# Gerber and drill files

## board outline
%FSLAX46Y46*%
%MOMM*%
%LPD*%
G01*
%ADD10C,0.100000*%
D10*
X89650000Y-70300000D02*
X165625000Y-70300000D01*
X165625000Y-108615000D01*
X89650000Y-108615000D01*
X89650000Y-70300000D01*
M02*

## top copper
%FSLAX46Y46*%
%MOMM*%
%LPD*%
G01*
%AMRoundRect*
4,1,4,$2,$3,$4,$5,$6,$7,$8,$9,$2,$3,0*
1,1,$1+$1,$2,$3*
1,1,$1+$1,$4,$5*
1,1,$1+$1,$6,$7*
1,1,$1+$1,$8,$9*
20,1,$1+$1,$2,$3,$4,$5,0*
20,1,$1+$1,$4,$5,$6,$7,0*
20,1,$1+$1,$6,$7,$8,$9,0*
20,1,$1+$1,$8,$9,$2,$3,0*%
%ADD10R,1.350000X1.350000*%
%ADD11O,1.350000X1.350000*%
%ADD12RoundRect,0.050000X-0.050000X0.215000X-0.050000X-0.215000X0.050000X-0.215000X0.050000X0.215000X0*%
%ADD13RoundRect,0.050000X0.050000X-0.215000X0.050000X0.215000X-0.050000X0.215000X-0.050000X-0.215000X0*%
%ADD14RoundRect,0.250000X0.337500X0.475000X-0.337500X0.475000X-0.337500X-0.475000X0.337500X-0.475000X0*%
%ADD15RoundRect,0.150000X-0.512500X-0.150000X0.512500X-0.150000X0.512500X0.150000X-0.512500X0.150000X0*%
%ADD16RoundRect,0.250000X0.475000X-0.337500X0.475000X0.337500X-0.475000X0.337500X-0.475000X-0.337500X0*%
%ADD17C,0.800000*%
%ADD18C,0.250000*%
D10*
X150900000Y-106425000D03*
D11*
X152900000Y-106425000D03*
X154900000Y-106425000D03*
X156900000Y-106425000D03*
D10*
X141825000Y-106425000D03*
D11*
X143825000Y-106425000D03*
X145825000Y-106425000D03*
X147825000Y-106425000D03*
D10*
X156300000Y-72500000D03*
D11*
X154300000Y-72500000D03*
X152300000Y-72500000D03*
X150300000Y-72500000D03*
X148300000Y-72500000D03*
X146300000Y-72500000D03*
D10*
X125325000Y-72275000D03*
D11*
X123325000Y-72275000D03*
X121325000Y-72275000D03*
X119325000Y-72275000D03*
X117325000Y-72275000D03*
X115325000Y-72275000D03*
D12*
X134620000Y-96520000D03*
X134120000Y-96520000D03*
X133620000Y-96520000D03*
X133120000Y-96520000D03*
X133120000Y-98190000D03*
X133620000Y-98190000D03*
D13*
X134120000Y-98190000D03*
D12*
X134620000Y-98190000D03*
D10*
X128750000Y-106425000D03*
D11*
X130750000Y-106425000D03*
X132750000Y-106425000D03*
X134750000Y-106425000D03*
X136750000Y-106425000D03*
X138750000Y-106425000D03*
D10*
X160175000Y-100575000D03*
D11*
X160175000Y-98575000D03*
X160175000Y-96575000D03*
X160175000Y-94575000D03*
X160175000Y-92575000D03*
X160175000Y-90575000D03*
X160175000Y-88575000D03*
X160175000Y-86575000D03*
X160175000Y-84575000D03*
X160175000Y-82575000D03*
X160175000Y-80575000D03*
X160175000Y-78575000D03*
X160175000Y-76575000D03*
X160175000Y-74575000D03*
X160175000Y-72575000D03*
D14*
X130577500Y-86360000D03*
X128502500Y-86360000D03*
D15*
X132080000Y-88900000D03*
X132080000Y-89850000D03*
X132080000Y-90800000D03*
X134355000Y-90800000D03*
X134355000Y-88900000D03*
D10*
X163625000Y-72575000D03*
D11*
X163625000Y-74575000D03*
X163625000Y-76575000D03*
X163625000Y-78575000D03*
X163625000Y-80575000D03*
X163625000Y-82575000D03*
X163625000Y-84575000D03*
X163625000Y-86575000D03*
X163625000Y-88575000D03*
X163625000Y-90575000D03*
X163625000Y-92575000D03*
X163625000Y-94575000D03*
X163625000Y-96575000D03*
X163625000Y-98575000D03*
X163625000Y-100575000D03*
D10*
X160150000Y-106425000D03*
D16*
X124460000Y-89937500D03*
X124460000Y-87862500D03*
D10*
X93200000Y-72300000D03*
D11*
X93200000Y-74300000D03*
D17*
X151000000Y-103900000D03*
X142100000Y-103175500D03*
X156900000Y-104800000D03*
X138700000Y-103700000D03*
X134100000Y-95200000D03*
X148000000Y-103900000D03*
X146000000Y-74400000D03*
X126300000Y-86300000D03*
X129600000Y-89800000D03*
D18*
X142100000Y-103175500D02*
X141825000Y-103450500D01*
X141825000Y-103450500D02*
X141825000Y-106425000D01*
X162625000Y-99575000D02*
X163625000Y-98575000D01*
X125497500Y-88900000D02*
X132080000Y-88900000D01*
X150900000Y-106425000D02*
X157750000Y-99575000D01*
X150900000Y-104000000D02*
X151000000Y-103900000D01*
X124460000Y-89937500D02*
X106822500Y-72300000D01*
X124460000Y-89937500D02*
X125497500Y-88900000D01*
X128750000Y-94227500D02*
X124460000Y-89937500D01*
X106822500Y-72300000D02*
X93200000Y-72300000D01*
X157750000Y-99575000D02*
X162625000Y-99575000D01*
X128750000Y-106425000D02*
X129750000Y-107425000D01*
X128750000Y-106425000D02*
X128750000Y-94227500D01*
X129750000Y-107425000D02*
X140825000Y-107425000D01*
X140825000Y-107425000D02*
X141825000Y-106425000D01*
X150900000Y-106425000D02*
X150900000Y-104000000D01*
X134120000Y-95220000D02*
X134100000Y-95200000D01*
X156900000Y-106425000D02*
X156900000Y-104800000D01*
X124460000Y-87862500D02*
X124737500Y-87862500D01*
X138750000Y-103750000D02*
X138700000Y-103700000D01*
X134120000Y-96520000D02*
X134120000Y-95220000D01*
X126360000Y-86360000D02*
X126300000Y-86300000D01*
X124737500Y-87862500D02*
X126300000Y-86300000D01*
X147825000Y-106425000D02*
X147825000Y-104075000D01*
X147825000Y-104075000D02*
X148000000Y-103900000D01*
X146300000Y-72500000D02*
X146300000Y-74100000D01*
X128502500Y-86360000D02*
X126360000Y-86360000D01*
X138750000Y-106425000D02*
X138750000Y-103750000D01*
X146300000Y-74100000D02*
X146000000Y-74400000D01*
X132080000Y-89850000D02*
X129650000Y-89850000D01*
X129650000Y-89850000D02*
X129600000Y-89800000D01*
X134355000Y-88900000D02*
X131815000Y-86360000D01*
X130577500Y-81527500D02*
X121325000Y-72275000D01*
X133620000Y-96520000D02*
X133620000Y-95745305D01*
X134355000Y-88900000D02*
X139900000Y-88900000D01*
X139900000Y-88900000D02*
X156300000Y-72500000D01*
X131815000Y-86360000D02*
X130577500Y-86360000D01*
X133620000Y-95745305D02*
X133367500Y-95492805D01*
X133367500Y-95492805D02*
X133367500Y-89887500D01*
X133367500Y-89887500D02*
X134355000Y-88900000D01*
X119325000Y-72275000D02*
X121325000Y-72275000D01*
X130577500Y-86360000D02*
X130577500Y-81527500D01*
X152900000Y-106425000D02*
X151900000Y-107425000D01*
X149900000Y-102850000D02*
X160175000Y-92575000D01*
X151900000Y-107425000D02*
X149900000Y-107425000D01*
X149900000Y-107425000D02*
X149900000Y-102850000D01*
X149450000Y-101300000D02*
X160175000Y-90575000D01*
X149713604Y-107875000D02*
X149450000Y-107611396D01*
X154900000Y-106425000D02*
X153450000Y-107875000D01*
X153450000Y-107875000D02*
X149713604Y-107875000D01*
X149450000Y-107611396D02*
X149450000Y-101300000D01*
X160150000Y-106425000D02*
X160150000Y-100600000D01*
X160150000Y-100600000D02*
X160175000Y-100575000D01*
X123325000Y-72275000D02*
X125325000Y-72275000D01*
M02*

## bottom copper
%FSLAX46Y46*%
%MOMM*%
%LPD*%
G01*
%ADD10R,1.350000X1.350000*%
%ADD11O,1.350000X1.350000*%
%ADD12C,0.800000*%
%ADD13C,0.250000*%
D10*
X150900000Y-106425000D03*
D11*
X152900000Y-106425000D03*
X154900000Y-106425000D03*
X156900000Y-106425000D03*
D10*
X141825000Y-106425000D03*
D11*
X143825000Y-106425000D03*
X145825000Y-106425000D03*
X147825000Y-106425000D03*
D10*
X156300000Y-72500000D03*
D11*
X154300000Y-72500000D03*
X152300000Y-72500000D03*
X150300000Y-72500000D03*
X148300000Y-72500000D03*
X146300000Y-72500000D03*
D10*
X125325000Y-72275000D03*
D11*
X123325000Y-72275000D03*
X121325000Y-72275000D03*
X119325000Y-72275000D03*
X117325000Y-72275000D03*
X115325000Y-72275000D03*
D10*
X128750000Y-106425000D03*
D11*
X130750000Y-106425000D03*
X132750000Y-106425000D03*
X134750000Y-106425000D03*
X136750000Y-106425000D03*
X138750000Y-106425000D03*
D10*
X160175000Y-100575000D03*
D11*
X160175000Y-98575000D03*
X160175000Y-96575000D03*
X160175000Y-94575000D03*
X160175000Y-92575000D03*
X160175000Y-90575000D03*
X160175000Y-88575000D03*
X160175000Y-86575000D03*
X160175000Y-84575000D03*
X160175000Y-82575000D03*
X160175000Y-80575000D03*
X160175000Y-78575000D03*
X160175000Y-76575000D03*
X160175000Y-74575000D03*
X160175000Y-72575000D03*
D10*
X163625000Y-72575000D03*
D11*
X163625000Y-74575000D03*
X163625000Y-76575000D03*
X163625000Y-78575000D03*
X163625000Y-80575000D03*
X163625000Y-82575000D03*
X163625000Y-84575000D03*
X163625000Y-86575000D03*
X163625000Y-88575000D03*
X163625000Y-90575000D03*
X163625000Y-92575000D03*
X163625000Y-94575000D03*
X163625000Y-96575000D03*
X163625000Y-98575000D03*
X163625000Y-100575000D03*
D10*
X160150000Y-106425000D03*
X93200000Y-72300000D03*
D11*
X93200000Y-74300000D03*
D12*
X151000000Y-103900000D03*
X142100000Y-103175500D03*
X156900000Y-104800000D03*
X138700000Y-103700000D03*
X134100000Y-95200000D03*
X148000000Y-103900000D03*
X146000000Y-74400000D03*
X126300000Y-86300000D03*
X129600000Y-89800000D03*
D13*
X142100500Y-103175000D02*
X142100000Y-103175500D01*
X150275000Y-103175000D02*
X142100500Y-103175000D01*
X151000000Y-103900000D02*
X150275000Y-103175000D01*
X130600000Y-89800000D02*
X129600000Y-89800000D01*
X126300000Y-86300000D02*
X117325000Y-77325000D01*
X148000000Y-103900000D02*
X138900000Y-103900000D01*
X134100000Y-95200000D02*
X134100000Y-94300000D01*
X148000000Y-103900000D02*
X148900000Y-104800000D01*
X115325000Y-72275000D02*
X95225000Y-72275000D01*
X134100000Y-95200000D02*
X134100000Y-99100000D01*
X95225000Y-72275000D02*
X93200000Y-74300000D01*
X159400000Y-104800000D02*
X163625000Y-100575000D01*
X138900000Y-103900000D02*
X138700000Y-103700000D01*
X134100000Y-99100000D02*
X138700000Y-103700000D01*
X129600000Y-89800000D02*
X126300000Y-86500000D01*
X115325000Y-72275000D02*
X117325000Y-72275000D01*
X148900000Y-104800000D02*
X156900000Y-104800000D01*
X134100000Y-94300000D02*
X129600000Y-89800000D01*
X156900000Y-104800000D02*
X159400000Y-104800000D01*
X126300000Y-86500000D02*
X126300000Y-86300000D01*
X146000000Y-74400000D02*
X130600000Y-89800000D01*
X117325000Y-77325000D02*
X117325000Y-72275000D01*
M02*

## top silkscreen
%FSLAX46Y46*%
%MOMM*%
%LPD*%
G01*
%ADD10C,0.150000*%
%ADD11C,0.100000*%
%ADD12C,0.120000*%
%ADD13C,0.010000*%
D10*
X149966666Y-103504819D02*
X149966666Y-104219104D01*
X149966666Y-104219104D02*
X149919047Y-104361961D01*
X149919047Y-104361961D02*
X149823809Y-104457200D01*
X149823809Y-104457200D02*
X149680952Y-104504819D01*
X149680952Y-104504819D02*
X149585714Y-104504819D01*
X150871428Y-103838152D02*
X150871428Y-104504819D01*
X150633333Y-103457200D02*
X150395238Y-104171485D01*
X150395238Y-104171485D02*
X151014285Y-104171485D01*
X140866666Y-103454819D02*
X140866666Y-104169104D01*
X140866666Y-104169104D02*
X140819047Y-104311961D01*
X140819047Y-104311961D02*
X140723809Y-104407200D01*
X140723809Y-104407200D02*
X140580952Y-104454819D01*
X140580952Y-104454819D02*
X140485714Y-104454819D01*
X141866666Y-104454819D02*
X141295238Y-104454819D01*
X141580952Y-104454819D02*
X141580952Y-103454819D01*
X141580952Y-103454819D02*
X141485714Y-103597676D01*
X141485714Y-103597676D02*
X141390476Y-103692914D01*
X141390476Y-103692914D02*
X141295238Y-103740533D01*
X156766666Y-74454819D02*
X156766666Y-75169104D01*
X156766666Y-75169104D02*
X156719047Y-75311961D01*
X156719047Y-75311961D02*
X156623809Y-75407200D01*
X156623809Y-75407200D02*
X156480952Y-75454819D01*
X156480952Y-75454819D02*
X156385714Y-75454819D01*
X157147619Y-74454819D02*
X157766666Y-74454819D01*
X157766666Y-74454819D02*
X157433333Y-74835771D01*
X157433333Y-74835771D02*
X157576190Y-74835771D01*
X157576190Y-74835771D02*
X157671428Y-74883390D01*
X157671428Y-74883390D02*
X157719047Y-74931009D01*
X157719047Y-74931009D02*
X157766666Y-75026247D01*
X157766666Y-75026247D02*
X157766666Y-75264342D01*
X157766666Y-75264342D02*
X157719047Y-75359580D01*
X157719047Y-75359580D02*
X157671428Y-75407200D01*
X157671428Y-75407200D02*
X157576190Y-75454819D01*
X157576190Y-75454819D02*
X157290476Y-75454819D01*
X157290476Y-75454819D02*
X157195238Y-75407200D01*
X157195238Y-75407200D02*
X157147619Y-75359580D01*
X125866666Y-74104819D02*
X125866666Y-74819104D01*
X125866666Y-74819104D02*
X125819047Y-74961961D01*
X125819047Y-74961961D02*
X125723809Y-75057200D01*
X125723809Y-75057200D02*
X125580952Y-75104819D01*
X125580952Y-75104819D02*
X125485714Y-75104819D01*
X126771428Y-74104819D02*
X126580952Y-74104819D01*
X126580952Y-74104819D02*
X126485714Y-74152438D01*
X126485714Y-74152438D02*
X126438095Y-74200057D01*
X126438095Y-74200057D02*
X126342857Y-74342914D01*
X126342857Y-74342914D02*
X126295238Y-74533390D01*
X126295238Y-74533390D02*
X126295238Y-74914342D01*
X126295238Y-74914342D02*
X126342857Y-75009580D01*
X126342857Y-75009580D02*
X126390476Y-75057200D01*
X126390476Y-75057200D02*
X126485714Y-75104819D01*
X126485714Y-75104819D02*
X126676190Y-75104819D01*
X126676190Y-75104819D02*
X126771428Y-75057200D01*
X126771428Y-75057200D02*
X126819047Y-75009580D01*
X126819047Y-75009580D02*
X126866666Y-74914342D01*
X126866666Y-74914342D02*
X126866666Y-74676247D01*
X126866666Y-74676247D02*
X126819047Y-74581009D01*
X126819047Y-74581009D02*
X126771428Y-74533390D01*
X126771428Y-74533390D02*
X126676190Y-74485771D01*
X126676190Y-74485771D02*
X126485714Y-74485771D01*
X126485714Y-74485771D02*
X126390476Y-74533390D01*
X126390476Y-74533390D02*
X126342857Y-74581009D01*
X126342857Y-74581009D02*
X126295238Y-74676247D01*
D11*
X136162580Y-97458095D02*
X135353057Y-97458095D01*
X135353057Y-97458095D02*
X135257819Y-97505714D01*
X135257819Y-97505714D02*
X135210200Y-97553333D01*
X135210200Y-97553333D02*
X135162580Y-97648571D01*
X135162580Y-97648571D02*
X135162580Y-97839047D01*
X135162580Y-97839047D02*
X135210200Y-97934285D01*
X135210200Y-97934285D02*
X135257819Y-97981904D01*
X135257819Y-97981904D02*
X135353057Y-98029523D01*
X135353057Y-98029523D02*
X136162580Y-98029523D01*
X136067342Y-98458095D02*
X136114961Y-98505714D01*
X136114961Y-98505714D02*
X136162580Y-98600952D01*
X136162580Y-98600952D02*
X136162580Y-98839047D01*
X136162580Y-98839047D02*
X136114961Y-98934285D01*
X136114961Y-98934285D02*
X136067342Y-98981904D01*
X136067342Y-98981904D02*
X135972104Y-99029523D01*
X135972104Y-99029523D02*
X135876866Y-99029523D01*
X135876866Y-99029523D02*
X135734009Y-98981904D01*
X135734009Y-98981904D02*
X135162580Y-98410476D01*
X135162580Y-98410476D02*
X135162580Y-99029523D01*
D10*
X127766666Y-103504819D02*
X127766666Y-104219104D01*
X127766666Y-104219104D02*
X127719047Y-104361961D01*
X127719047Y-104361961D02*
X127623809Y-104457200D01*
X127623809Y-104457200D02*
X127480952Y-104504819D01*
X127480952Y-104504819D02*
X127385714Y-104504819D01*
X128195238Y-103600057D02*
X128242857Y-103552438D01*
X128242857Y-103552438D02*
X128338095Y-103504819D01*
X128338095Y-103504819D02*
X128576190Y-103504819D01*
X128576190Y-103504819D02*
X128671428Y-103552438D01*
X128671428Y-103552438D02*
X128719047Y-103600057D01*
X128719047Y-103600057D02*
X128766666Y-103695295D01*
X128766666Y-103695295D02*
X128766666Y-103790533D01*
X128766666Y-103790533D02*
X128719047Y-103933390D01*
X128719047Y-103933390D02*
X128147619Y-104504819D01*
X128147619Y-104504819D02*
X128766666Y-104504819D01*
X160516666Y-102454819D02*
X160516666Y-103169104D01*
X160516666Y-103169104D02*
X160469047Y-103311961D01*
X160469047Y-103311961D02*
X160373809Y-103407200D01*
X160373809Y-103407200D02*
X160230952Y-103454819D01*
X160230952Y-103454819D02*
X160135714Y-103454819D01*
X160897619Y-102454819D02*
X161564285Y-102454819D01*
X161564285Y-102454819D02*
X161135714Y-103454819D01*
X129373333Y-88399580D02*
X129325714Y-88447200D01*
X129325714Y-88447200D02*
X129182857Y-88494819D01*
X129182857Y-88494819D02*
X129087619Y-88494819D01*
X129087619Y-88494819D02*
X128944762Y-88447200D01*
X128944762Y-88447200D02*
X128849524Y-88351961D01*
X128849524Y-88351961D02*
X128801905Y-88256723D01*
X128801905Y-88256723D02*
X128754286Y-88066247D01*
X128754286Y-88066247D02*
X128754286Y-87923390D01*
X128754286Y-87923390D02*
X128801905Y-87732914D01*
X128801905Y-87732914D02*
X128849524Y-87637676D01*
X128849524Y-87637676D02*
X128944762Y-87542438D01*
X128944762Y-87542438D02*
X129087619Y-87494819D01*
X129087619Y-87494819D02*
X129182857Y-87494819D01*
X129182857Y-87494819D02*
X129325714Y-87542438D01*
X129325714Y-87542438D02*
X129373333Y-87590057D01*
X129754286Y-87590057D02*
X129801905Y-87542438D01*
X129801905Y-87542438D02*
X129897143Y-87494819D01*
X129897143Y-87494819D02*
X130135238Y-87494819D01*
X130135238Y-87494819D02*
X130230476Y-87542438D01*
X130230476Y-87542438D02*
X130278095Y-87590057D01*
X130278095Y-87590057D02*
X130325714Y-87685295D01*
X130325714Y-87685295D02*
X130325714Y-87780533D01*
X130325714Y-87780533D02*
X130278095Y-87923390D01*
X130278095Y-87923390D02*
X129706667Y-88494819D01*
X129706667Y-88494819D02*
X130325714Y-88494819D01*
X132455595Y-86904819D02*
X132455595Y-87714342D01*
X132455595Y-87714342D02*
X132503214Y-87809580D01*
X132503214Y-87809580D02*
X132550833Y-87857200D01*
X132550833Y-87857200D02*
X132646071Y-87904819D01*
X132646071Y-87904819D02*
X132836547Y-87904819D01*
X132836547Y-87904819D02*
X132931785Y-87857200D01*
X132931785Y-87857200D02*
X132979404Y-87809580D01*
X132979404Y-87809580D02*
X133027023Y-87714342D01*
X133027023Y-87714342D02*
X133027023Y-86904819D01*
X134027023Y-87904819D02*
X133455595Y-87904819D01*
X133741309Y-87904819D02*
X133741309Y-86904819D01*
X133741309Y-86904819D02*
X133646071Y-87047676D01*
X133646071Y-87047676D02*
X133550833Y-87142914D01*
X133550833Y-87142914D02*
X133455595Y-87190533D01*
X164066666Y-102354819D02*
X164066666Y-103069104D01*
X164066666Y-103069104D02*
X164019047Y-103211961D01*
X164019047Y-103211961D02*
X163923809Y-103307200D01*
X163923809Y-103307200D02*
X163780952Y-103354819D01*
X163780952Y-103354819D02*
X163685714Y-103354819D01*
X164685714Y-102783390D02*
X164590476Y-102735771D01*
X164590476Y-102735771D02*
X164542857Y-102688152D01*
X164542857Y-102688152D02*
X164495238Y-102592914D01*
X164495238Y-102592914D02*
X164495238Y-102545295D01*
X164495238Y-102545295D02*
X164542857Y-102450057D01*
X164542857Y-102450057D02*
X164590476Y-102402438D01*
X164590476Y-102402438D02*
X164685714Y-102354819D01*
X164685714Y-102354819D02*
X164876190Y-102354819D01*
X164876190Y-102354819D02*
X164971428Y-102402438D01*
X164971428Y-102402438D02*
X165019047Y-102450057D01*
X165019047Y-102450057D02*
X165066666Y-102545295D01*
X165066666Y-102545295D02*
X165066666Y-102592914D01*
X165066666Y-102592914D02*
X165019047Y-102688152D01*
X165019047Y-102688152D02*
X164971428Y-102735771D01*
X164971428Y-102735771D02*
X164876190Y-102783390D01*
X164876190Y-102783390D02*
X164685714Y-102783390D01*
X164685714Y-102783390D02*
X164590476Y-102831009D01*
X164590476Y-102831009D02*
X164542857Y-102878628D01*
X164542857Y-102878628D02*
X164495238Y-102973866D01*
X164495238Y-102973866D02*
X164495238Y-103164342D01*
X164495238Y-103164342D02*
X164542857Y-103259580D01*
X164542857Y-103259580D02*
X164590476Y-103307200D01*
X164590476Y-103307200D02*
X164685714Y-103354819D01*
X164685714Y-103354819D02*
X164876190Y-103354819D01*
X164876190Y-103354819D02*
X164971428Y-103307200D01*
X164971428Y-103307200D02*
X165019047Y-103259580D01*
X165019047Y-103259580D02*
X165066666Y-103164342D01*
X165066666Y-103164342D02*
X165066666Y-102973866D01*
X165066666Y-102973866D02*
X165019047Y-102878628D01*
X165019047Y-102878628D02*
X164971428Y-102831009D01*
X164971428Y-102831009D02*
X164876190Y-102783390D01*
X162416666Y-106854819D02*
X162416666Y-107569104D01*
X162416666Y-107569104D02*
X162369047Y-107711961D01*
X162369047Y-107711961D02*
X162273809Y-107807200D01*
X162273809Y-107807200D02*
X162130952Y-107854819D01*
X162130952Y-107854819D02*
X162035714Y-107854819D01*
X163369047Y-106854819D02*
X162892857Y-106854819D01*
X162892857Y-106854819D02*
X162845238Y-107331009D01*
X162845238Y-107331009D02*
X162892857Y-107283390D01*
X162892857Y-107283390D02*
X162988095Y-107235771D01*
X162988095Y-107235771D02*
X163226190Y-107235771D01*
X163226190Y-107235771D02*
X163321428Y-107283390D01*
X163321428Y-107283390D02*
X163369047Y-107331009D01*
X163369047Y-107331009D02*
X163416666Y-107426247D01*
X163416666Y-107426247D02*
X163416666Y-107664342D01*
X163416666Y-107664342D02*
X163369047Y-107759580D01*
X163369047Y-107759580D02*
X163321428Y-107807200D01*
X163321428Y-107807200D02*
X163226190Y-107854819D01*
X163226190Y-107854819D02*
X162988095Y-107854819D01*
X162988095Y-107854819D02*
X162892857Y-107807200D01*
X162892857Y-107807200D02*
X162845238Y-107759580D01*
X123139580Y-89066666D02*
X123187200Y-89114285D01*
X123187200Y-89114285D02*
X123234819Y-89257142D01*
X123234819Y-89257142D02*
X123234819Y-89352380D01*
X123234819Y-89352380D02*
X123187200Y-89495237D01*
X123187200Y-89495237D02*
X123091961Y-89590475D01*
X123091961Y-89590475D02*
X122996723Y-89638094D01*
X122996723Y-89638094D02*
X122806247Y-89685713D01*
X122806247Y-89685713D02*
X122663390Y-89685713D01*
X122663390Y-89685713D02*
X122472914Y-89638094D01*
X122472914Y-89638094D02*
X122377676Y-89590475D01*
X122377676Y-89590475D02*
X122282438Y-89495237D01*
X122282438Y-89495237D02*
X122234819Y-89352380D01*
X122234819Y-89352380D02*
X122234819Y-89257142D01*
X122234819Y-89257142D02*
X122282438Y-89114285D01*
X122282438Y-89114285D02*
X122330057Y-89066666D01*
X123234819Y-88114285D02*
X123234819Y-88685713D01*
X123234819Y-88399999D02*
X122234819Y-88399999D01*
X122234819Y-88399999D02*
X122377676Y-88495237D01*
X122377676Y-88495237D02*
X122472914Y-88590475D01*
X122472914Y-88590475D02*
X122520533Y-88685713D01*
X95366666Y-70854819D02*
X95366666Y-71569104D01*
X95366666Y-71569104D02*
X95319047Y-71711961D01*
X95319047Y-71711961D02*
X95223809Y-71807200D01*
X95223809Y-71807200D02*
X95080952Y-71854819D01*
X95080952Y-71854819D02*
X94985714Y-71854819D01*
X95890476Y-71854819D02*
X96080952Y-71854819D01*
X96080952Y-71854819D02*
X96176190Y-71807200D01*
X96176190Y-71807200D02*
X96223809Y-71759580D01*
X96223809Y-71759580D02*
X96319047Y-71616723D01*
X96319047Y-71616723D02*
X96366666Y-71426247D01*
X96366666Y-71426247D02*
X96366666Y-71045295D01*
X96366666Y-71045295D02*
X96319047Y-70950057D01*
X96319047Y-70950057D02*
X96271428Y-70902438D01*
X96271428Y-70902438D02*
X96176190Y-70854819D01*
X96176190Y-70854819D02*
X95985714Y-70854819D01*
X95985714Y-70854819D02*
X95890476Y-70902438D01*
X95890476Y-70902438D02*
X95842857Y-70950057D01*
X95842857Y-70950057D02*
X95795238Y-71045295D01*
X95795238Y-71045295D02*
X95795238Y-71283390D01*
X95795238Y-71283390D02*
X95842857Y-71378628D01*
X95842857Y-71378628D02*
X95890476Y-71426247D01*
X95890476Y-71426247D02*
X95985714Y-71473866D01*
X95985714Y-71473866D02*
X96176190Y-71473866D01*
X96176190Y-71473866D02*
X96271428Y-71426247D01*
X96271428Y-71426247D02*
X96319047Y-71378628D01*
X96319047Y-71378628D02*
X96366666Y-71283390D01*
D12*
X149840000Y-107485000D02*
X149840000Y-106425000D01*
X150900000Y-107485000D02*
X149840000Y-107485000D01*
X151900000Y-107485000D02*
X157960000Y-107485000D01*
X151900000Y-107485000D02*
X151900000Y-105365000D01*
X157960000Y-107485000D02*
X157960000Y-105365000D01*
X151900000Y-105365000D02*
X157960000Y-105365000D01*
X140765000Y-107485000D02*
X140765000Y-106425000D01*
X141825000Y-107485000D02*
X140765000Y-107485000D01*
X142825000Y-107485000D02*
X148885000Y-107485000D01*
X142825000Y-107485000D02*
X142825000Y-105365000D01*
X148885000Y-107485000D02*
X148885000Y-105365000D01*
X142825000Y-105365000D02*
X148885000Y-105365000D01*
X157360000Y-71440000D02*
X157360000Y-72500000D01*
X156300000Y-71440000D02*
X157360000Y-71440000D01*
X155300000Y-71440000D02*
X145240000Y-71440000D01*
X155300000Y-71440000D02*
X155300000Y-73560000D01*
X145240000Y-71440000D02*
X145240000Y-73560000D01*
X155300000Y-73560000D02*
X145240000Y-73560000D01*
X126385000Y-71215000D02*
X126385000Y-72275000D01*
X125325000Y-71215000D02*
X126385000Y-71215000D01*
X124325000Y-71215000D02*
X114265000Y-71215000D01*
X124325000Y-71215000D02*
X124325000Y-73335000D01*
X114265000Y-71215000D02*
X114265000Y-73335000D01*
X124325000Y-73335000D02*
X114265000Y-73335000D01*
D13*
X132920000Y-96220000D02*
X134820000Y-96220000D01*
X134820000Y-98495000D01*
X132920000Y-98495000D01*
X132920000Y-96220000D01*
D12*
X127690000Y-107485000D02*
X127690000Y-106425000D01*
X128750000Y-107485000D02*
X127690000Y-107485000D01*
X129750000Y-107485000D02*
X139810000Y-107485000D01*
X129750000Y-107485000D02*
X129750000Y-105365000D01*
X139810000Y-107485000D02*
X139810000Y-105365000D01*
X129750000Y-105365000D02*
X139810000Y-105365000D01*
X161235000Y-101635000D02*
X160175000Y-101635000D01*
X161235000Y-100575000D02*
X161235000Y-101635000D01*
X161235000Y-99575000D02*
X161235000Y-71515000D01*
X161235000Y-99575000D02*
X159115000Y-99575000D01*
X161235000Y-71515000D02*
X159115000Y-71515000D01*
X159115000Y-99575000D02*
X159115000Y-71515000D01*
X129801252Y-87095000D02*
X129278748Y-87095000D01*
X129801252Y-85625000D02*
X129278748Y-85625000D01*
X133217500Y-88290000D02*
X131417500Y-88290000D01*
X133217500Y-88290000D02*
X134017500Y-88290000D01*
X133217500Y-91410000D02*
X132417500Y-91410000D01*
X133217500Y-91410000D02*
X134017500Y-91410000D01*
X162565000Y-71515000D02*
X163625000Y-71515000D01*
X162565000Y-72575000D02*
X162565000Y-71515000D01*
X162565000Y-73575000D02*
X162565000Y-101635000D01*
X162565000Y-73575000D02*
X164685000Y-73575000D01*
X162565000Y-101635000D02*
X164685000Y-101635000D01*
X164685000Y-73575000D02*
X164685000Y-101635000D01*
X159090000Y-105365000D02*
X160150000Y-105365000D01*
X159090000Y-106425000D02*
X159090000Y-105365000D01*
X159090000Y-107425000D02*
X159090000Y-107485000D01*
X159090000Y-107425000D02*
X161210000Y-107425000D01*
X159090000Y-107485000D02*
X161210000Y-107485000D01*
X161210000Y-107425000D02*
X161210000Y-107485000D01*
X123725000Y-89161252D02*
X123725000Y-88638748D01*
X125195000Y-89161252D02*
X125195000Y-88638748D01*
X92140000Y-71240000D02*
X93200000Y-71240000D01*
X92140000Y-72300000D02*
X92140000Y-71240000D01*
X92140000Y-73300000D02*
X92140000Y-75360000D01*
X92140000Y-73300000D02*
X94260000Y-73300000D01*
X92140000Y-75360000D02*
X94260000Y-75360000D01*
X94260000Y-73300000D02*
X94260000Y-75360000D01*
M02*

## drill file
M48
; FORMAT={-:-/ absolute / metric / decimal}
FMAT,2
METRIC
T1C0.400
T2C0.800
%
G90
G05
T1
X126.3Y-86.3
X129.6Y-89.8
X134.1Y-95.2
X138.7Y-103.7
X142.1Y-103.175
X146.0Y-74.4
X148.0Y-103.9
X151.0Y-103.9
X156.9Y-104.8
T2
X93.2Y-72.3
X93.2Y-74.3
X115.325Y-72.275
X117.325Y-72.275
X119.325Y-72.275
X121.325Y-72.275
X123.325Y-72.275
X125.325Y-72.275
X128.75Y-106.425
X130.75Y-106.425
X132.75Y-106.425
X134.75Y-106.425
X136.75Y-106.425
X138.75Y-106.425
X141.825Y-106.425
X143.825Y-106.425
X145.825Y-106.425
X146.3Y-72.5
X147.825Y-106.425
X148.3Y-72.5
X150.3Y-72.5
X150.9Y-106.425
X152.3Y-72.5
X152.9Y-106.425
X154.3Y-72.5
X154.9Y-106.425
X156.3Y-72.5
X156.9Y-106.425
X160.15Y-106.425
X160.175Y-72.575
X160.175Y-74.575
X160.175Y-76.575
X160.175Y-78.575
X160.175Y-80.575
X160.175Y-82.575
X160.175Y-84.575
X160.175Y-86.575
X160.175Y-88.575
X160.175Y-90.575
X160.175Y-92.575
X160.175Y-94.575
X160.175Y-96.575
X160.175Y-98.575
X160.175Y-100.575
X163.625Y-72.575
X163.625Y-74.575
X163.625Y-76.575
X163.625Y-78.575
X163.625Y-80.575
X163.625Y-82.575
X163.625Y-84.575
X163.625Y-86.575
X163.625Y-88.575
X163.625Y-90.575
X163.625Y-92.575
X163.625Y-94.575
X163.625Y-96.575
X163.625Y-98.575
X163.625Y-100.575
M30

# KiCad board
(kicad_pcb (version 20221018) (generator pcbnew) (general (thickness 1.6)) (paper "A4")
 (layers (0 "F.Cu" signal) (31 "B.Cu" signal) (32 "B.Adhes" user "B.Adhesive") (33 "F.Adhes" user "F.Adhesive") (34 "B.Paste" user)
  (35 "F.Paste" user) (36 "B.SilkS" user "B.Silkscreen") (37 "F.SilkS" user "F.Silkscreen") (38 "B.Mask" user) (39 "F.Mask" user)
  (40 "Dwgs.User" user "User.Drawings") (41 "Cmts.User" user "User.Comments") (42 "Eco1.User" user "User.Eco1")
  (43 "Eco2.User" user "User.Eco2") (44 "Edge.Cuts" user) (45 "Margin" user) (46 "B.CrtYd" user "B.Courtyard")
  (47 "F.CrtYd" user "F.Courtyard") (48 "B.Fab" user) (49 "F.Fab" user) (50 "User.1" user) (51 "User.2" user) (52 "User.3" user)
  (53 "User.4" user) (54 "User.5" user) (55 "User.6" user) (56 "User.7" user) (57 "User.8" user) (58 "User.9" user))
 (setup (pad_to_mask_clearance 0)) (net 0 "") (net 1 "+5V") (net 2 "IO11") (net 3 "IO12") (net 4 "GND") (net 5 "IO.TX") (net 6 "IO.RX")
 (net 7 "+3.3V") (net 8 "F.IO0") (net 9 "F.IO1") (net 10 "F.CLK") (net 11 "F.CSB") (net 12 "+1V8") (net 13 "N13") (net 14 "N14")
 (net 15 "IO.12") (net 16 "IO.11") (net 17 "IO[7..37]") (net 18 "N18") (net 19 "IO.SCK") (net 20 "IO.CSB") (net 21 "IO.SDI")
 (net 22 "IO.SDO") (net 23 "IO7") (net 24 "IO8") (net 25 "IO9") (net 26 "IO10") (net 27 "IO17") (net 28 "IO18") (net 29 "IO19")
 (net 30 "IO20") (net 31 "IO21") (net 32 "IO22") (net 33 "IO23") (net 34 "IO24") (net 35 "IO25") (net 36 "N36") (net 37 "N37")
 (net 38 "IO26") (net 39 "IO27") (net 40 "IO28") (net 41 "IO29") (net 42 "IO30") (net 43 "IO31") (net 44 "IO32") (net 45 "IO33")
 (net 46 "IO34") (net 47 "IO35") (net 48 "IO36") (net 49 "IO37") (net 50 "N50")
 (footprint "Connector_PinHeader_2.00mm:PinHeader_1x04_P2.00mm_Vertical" (layer "F.Cu") (at 150.9 106.425 90)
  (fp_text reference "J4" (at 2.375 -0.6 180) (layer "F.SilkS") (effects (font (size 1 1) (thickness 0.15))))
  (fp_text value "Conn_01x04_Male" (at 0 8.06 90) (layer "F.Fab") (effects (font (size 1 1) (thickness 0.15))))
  (fp_line (start -1.06 -1.06) (end 0 -1.06) (stroke (width 0.12) (type solid)) (layer "F.SilkS"))
  (fp_line (start -1.06 0) (end -1.06 -1.06) (stroke (width 0.12) (type solid)) (layer "F.SilkS"))
  (fp_line (start -1.06 1) (end -1.06 7.06) (stroke (width 0.12) (type solid)) (layer "F.SilkS"))
  (fp_line (start -1.06 1) (end 1.06 1) (stroke (width 0.12) (type solid)) (layer "F.SilkS"))
  (fp_line (start -1.06 7.06) (end 1.06 7.06) (stroke (width 0.12) (type solid)) (layer "F.SilkS"))
  (fp_line (start 1.06 1) (end 1.06 7.06) (stroke (width 0.12) (type solid)) (layer "F.SilkS"))
  (pad "1" thru_hole rect (at 0 0 90) (size 1.35 1.35) (drill 0.8) (layers "*.Cu" "*.Mask") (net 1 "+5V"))
  (pad "2" thru_hole oval (at 0 2 90) (size 1.35 1.35) (drill 0.8) (layers "*.Cu" "*.Mask") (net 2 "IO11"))
  (pad "3" thru_hole oval (at 0 4 90) (size 1.35 1.35) (drill 0.8) (layers "*.Cu" "*.Mask") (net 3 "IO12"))
  (pad "4" thru_hole oval (at 0 6 90) (size 1.35 1.35) (drill 0.8) (layers "*.Cu" "*.Mask") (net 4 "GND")))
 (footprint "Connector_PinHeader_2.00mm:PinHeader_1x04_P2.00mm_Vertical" (layer "F.Cu") (at 141.825 106.425 90)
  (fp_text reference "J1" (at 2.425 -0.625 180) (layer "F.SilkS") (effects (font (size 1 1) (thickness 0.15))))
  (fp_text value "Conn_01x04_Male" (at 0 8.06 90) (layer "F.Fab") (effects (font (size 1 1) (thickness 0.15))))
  (fp_line (start -1.06 -1.06) (end 0 -1.06) (stroke (width 0.12) (type solid)) (layer "F.SilkS"))
  (fp_line (start -1.06 0) (end -1.06 -1.06) (stroke (width 0.12) (type solid)) (layer "F.SilkS"))
  (fp_line (start -1.06 1) (end -1.06 7.06) (stroke (width 0.12) (type solid)) (layer "F.SilkS"))
  (fp_line (start -1.06 1) (end 1.06 1) (stroke (width 0.12) (type solid)) (layer "F.SilkS"))
  (fp_line (start -1.06 7.06) (end 1.06 7.06) (stroke (width 0.12) (type solid)) (layer "F.SilkS"))
  (fp_line (start 1.06 1) (end 1.06 7.06) (stroke (width 0.12) (type solid)) (layer "F.SilkS"))
  (pad "1" thru_hole rect (at 0 0 90) (size 1.35 1.35) (drill 0.8) (layers "*.Cu" "*.Mask") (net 1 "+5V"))
  (pad "2" thru_hole oval (at 0 2 90) (size 1.35 1.35) (drill 0.8) (layers "*.Cu" "*.Mask") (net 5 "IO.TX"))
  (pad "3" thru_hole oval (at 0 4 90) (size 1.35 1.35) (drill 0.8) (layers "*.Cu" "*.Mask") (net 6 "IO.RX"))
  (pad "4" thru_hole oval (at 0 6 90) (size 1.35 1.35) (drill 0.8) (layers "*.Cu" "*.Mask") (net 4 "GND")))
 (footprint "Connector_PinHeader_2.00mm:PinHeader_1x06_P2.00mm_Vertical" (layer "F.Cu") (at 156.3 72.5 -90)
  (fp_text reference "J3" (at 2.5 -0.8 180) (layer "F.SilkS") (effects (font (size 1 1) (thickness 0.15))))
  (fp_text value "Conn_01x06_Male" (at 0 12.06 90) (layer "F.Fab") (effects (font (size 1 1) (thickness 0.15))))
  (fp_line (start -1.06 -1.06) (end 0 -1.06) (stroke (width 0.12) (type solid)) (layer "F.SilkS"))
  (fp_line (start -1.06 0) (end -1.06 -1.06) (stroke (width 0.12) (type solid)) (layer "F.SilkS"))
  (fp_line (start -1.06 1) (end -1.06 11.06) (stroke (width 0.12) (type solid)) (layer "F.SilkS"))
  (fp_line (start -1.06 1) (end 1.06 1) (stroke (width 0.12) (type solid)) (layer "F.SilkS"))
  (fp_line (start -1.06 11.06) (end 1.06 11.06) (stroke (width 0.12) (type solid)) (layer "F.SilkS"))
  (fp_line (start 1.06 1) (end 1.06 11.06) (stroke (width 0.12) (type solid)) (layer "F.SilkS"))
  (pad "1" thru_hole rect (at 0 0 270) (size 1.35 1.35) (drill 0.8) (layers "*.Cu" "*.Mask") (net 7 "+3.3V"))
  (pad "2" thru_hole oval (at 0 2 270) (size 1.35 1.35) (drill 0.8) (layers "*.Cu" "*.Mask") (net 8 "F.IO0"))
  (pad "3" thru_hole oval (at 0 4 270) (size 1.35 1.35) (drill 0.8) (layers "*.Cu" "*.Mask") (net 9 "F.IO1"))
  (pad "4" thru_hole oval (at 0 6 270) (size 1.35 1.35) (drill 0.8) (layers "*.Cu" "*.Mask") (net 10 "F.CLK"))
  (pad "5" thru_hole oval (at 0 8 270) (size 1.35 1.35) (drill 0.8) (layers "*.Cu" "*.Mask") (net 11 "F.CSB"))
  (pad "6" thru_hole oval (at 0 10 270) (size 1.35 1.35) (drill 0.8) (layers "*.Cu" "*.Mask") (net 4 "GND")))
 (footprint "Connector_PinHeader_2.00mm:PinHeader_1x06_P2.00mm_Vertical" (layer "F.Cu") (at 125.325 72.275 -90)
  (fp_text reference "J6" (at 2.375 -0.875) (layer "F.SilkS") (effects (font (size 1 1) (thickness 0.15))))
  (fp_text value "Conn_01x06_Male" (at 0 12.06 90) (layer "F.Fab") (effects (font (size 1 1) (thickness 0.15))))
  (fp_line (start -1.06 -1.06) (end 0 -1.06) (stroke (width 0.12) (type solid)) (layer "F.SilkS"))
  (fp_line (start -1.06 0) (end -1.06 -1.06) (stroke (width 0.12) (type solid)) (layer "F.SilkS"))
  (fp_line (start -1.06 1) (end -1.06 11.06) (stroke (width 0.12) (type solid)) (layer "F.SilkS"))
  (fp_line (start -1.06 1) (end 1.06 1) (stroke (width 0.12) (type solid)) (layer "F.SilkS"))
  (fp_line (start -1.06 11.06) (end 1.06 11.06) (stroke (width 0.12) (type solid)) (layer "F.SilkS"))
  (fp_line (start 1.06 1) (end 1.06 11.06) (stroke (width 0.12) (type solid)) (layer "F.SilkS"))
  (pad "1" thru_hole rect (at 0 0 270) (size 1.35 1.35) (drill 0.8) (layers "*.Cu" "*.Mask") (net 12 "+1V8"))
  (pad "2" thru_hole oval (at 0 2 270) (size 1.35 1.35) (drill 0.8) (layers "*.Cu" "*.Mask") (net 12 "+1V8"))
  (pad "3" thru_hole oval (at 0 4 270) (size 1.35 1.35) (drill 0.8) (layers "*.Cu" "*.Mask") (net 7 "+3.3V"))
  (pad "4" thru_hole oval (at 0 6 270) (size 1.35 1.35) (drill 0.8) (layers "*.Cu" "*.Mask") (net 7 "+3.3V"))
  (pad "5" thru_hole oval (at 0 8 270) (size 1.35 1.35) (drill 0.8) (layers "*.Cu" "*.Mask") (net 4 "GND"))
  (pad "6" thru_hole oval (at 0 10 270) (size 1.35 1.35) (drill 0.8) (layers "*.Cu" "*.Mask") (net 4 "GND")))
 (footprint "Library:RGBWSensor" (layer "F.Cu") (at 133.02 96.32 -90)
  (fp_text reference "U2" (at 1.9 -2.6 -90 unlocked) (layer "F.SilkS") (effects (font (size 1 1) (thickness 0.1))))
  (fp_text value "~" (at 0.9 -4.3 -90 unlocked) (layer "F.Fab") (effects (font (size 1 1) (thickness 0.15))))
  (fp_rect (start -0.1 -1.8) (end 2.175 0.1) (stroke (width 0.01) (type default)) (fill none) (layer "F.SilkS"))
  (pad "1" smd roundrect (at 0.2 -1.6 270) (size 0.53 0.2) (layers "F.Cu" "F.Paste" "F.Mask") (roundrect_rratio 0.25) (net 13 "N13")
   (thermal_bridge_angle 45))
  (pad "2" smd roundrect (at 0.2 -1.1 270) (size 0.53 0.2) (layers "F.Cu" "F.Paste" "F.Mask") (roundrect_rratio 0.25) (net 4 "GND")
   (thermal_bridge_angle 45))
  (pad "3" smd roundrect (at 0.2 -0.6 270) (size 0.53 0.2) (layers "F.Cu" "F.Paste" "F.Mask") (roundrect_rratio 0.25) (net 7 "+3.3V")
   (thermal_bridge_angle 45))
  (pad "4" smd roundrect (at 0.2 -0.1 270) (size 0.53 0.2) (layers "F.Cu" "F.Paste" "F.Mask") (roundrect_rratio 0.25) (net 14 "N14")
   (thermal_bridge_angle 45))
  (pad "5" smd roundrect (at 1.87 -0.1 270) (size 0.53 0.2) (layers "F.Cu" "F.Paste" "F.Mask") (roundrect_rratio 0.25) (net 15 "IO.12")
   (thermal_bridge_angle 45))
  (pad "6" smd roundrect (at 1.87 -0.6 270) (size 0.53 0.2) (layers "F.Cu" "F.Paste" "F.Mask") (roundrect_rratio 0.25) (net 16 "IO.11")
   (thermal_bridge_angle 45))
  (pad "7" smd roundrect (at 1.87 -1.1 90) (size 0.53 0.2) (layers "F.Cu" "F.Paste" "F.Mask") (roundrect_rratio 0.25) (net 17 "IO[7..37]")
   (thermal_bridge_angle 45))
  (pad "8" smd roundrect (at 1.87 -1.6 270) (size 0.53 0.2) (layers "F.Cu" "F.Paste" "F.Mask") (roundrect_rratio 0.25) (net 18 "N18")
   (thermal_bridge_angle 45)))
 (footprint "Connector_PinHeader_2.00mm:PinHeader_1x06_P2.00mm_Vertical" (layer "F.Cu") (at 128.75 106.425 90)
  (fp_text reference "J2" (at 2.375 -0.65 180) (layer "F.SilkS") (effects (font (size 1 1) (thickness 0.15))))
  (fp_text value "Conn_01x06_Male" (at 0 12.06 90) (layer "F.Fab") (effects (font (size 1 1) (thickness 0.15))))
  (fp_line (start -1.06 -1.06) (end 0 -1.06) (stroke (width 0.12) (type solid)) (layer "F.SilkS"))
  (fp_line (start -1.06 0) (end -1.06 -1.06) (stroke (width 0.12) (type solid)) (layer "F.SilkS"))
  (fp_line (start -1.06 1) (end -1.06 11.06) (stroke (width 0.12) (type solid)) (layer "F.SilkS"))
  (fp_line (start -1.06 1) (end 1.06 1) (stroke (width 0.12) (type solid)) (layer "F.SilkS"))
  (fp_line (start -1.06 11.06) (end 1.06 11.06) (stroke (width 0.12) (type solid)) (layer "F.SilkS"))
  (fp_line (start 1.06 1) (end 1.06 11.06) (stroke (width 0.12) (type solid)) (layer "F.SilkS"))
  (pad "1" thru_hole rect (at 0 0 90) (size 1.35 1.35) (drill 0.8) (layers "*.Cu" "*.Mask") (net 1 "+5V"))
  (pad "2" thru_hole oval (at 0 2 90) (size 1.35 1.35) (drill 0.8) (layers "*.Cu" "*.Mask") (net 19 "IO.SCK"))
  (pad "3" thru_hole oval (at 0 4 90) (size 1.35 1.35) (drill 0.8) (layers "*.Cu" "*.Mask") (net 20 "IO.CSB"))
  (pad "4" thru_hole oval (at 0 6 90) (size 1.35 1.35) (drill 0.8) (layers "*.Cu" "*.Mask") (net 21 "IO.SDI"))
  (pad "5" thru_hole oval (at 0 8 90) (size 1.35 1.35) (drill 0.8) (layers "*.Cu" "*.Mask") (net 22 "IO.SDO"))
  (pad "6" thru_hole oval (at 0 10 90) (size 1.35 1.35) (drill 0.8) (layers "*.Cu" "*.Mask") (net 4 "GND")))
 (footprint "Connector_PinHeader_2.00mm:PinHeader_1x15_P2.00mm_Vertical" (layer "F.Cu") (at 160.175 100.575 180)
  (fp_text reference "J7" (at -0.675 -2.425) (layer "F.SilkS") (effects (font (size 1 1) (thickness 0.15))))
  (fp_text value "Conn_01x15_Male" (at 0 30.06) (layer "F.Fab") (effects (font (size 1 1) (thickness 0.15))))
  (fp_line (start -1.06 -1.06) (end 0 -1.06) (stroke (width 0.12) (type solid)) (layer "F.SilkS"))
  (fp_line (start -1.06 0) (end -1.06 -1.06) (stroke (width 0.12) (type solid)) (layer "F.SilkS"))
  (fp_line (start -1.06 1) (end -1.06 29.06) (stroke (width 0.12) (type solid)) (layer "F.SilkS"))
  (fp_line (start -1.06 1) (end 1.06 1) (stroke (width 0.12) (type solid)) (layer "F.SilkS"))
  (fp_line (start -1.06 29.06) (end 1.06 29.06) (stroke (width 0.12) (type solid)) (layer "F.SilkS"))
  (fp_line (start 1.06 1) (end 1.06 29.06) (stroke (width 0.12) (type solid)) (layer "F.SilkS"))
  (pad "1" thru_hole rect (at 0 0 180) (size 1.35 1.35) (drill 0.8) (layers "*.Cu" "*.Mask") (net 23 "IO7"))
  (pad "2" thru_hole oval (at 0 2 180) (size 1.35 1.35) (drill 0.8) (layers "*.Cu" "*.Mask") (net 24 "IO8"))
  (pad "3" thru_hole oval (at 0 4 180) (size 1.35 1.35) (drill 0.8) (layers "*.Cu" "*.Mask") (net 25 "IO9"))
  (pad "4" thru_hole oval (at 0 6 180) (size 1.35 1.35) (drill 0.8) (layers "*.Cu" "*.Mask") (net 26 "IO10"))
  (pad "5" thru_hole oval (at 0 8 180) (size 1.35 1.35) (drill 0.8) (layers "*.Cu" "*.Mask") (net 2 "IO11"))
  (pad "6" thru_hole oval (at 0 10 180) (size 1.35 1.35) (drill 0.8) (layers "*.Cu" "*.Mask") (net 3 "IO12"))
  (pad "7" thru_hole oval (at 0 12 180) (size 1.35 1.35) (drill 0.8) (layers "*.Cu" "*.Mask") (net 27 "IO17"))
  (pad "8" thru_hole oval (at 0 14 180) (size 1.35 1.35) (drill 0.8) (layers "*.Cu" "*.Mask") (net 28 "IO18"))
  (pad "9" thru_hole oval (at 0 16 180) (size 1.35 1.35) (drill 0.8) (layers "*.Cu" "*.Mask") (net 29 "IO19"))
  (pad "10" thru_hole oval (at 0 18 180) (size 1.35 1.35) (drill 0.8) (layers "*.Cu" "*.Mask") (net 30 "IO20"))
  (pad "11" thru_hole oval (at 0 20 180) (size 1.35 1.35) (drill 0.8) (layers "*.Cu" "*.Mask") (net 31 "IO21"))
  (pad "12" thru_hole oval (at 0 22 180) (size 1.35 1.35) (drill 0.8) (layers "*.Cu" "*.Mask") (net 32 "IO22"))
  (pad "13" thru_hole oval (at 0 24 180) (size 1.35 1.35) (drill 0.8) (layers "*.Cu" "*.Mask") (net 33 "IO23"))
  (pad "14" thru_hole oval (at 0 26 180) (size 1.35 1.35) (drill 0.8) (layers "*.Cu" "*.Mask") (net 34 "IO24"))
  (pad "15" thru_hole oval (at 0 28 180) (size 1.35 1.35) (drill 0.8) (layers "*.Cu" "*.Mask") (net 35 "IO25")))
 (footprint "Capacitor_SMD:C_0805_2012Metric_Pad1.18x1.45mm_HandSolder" (layer "F.Cu") (at 129.54 86.36 180)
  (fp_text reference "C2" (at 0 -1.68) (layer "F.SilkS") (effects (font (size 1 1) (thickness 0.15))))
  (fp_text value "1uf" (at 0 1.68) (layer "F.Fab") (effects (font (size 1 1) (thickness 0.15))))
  (fp_line (start -0.261252 -0.735) (end 0.261252 -0.735) (stroke (width 0.12) (type solid)) (layer "F.SilkS"))
  (fp_line (start -0.261252 0.735) (end 0.261252 0.735) (stroke (width 0.12) (type solid)) (layer "F.SilkS"))
  (pad "1" smd roundrect (at -1.0375 0 180) (size 1.175 1.45) (layers "F.Cu" "F.Paste" "F.Mask") (roundrect_rratio 0.212766) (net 7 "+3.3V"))
  (pad "2" smd roundrect (at 1.0375 0 180) (size 1.175 1.45) (layers "F.Cu" "F.Paste" "F.Mask") (roundrect_rratio 0.212766) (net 4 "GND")))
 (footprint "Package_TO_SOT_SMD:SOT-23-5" (layer "F.Cu") (at 133.2175 89.85)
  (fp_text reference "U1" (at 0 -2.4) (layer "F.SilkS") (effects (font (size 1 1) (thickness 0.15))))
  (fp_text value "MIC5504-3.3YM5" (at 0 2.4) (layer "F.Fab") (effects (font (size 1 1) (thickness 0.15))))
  (fp_line (start 0 -1.56) (end -1.8 -1.56) (stroke (width 0.12) (type solid)) (layer "F.SilkS"))
  (fp_line (start 0 -1.56) (end 0.8 -1.56) (stroke (width 0.12) (type solid)) (layer "F.SilkS"))
  (fp_line (start 0 1.56) (end -0.8 1.56) (stroke (width 0.12) (type solid)) (layer "F.SilkS"))
  (fp_line (start 0 1.56) (end 0.8 1.56) (stroke (width 0.12) (type solid)) (layer "F.SilkS"))
  (pad "1" smd roundrect (at -1.1375 -0.95) (size 1.325 0.6) (layers "F.Cu" "F.Paste" "F.Mask") (roundrect_rratio 0.25) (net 1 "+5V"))
  (pad "2" smd roundrect (at -1.1375 0) (size 1.325 0.6) (layers "F.Cu" "F.Paste" "F.Mask") (roundrect_rratio 0.25) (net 4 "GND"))
  (pad "3" smd roundrect (at -1.1375 0.95) (size 1.325 0.6) (layers "F.Cu" "F.Paste" "F.Mask") (roundrect_rratio 0.25) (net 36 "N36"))
  (pad "4" smd roundrect (at 1.1375 0.95) (size 1.325 0.6) (layers "F.Cu" "F.Paste" "F.Mask") (roundrect_rratio 0.25) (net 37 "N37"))
  (pad "5" smd roundrect (at 1.1375 -0.95) (size 1.325 0.6) (layers "F.Cu" "F.Paste" "F.Mask") (roundrect_rratio 0.25) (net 7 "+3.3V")))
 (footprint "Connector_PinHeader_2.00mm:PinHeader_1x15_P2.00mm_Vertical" (layer "F.Cu") (at 163.625 72.575)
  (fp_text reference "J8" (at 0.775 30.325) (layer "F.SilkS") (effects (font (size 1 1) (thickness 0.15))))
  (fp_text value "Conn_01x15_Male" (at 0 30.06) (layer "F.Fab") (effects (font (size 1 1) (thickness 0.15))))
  (fp_line (start -1.06 -1.06) (end 0 -1.06) (stroke (width 0.12) (type solid)) (layer "F.SilkS"))
  (fp_line (start -1.06 0) (end -1.06 -1.06) (stroke (width 0.12) (type solid)) (layer "F.SilkS"))
  (fp_line (start -1.06 1) (end -1.06 29.06) (stroke (width 0.12) (type solid)) (layer "F.SilkS"))
  (fp_line (start -1.06 1) (end 1.06 1) (stroke (width 0.12) (type solid)) (layer "F.SilkS"))
  (fp_line (start -1.06 29.06) (end 1.06 29.06) (stroke (width 0.12) (type solid)) (layer "F.SilkS"))
  (fp_line (start 1.06 1) (end 1.06 29.06) (stroke (width 0.12) (type solid)) (layer "F.SilkS"))
  (pad "1" thru_hole rect (at 0 0) (size 1.35 1.35) (drill 0.8) (layers "*.Cu" "*.Mask") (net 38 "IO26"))
  (pad "2" thru_hole oval (at 0 2) (size 1.35 1.35) (drill 0.8) (layers "*.Cu" "*.Mask") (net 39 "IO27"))
  (pad "3" thru_hole oval (at 0 4) (size 1.35 1.35) (drill 0.8) (layers "*.Cu" "*.Mask") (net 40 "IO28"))
  (pad "4" thru_hole oval (at 0 6) (size 1.35 1.35) (drill 0.8) (layers "*.Cu" "*.Mask") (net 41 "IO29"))
  (pad "5" thru_hole oval (at 0 8) (size 1.35 1.35) (drill 0.8) (layers "*.Cu" "*.Mask") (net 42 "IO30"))
  (pad "6" thru_hole oval (at 0 10) (size 1.35 1.35) (drill 0.8) (layers "*.Cu" "*.Mask") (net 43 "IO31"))
  (pad "7" thru_hole oval (at 0 12) (size 1.35 1.35) (drill 0.8) (layers "*.Cu" "*.Mask") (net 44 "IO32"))
  (pad "8" thru_hole oval (at 0 14) (size 1.35 1.35) (drill 0.8) (layers "*.Cu" "*.Mask") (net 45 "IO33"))
  (pad "9" thru_hole oval (at 0 16) (size 1.35 1.35) (drill 0.8) (layers "*.Cu" "*.Mask") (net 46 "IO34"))
  (pad "10" thru_hole oval (at 0 18) (size 1.35 1.35) (drill 0.8) (layers "*.Cu" "*.Mask") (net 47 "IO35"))
  (pad "11" thru_hole oval (at 0 20) (size 1.35 1.35) (drill 0.8) (layers "*.Cu" "*.Mask") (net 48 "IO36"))
  (pad "12" thru_hole oval (at 0 22) (size 1.35 1.35) (drill 0.8) (layers "*.Cu" "*.Mask") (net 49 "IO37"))
  (pad "13" thru_hole oval (at 0 24) (size 1.35 1.35) (drill 0.8) (layers "*.Cu" "*.Mask") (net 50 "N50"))
  (pad "14" thru_hole oval (at 0 26) (size 1.35 1.35) (drill 0.8) (layers "*.Cu" "*.Mask") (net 1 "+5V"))
  (pad "15" thru_hole oval (at 0 28) (size 1.35 1.35) (drill 0.8) (layers "*.Cu" "*.Mask") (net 4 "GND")))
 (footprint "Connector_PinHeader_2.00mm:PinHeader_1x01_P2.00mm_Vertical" (layer "F.Cu") (at 160.15 106.425)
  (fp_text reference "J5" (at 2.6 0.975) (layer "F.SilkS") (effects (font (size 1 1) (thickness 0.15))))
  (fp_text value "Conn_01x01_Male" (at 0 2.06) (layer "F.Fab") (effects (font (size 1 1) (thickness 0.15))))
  (fp_line (start -1.06 -1.06) (end 0 -1.06) (stroke (width 0.12) (type solid)) (layer "F.SilkS"))
  (fp_line (start -1.06 0) (end -1.06 -1.06) (stroke (width 0.12) (type solid)) (layer "F.SilkS"))
  (fp_line (start -1.06 1) (end -1.06 1.06) (stroke (width 0.12) (type solid)) (layer "F.SilkS"))
  (fp_line (start -1.06 1) (end 1.06 1) (stroke (width 0.12) (type solid)) (layer "F.SilkS"))
  (fp_line (start -1.06 1.06) (end 1.06 1.06) (stroke (width 0.12) (type solid)) (layer "F.SilkS"))
  (fp_line (start 1.06 1) (end 1.06 1.06) (stroke (width 0.12) (type solid)) (layer "F.SilkS"))
  (pad "1" thru_hole rect (at 0 0) (size 1.35 1.35) (drill 0.8) (layers "*.Cu" "*.Mask") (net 23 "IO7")))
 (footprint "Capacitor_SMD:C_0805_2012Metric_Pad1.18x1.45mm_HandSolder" (layer "F.Cu") (at 124.46 88.9 90)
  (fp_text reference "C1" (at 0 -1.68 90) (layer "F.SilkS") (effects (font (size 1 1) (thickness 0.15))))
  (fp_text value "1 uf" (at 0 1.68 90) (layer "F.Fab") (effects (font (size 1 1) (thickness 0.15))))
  (fp_line (start -0.261252 -0.735) (end 0.261252 -0.735) (stroke (width 0.12) (type solid)) (layer "F.SilkS"))
  (fp_line (start -0.261252 0.735) (end 0.261252 0.735) (stroke (width 0.12) (type solid)) (layer "F.SilkS"))
  (pad "1" smd roundrect (at -1.0375 0 90) (size 1.175 1.45) (layers "F.Cu" "F.Paste" "F.Mask") (roundrect_rratio 0.212766) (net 1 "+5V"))
  (pad "2" smd roundrect (at 1.0375 0 90) (size 1.175 1.45) (layers "F.Cu" "F.Paste" "F.Mask") (roundrect_rratio 0.212766) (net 4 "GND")))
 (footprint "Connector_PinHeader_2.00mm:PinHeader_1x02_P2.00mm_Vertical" (layer "F.Cu") (at 93.2 72.3)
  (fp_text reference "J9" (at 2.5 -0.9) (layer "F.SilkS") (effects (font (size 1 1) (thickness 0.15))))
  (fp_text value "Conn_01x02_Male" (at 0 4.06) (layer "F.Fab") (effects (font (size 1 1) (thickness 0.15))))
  (fp_line (start -1.06 -1.06) (end 0 -1.06) (stroke (width 0.12) (type solid)) (layer "F.SilkS"))
  (fp_line (start -1.06 0) (end -1.06 -1.06) (stroke (width 0.12) (type solid)) (layer "F.SilkS"))
  (fp_line (start -1.06 1) (end -1.06 3.06) (stroke (width 0.12) (type solid)) (layer "F.SilkS"))
  (fp_line (start -1.06 1) (end 1.06 1) (stroke (width 0.12) (type solid)) (layer "F.SilkS"))
  (fp_line (start -1.06 3.06) (end 1.06 3.06) (stroke (width 0.12) (type solid)) (layer "F.SilkS"))
  (fp_line (start 1.06 1) (end 1.06 3.06) (stroke (width 0.12) (type solid)) (layer "F.SilkS"))
  (pad "1" thru_hole rect (at 0 0) (size 1.35 1.35) (drill 0.8) (layers "*.Cu" "*.Mask") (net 1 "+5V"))
  (pad "2" thru_hole oval (at 0 2) (size 1.35 1.35) (drill 0.8) (layers "*.Cu" "*.Mask") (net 4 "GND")))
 (gr_rect (start 89.65 70.3) (end 165.625 108.615) (stroke (width 0.1) (type solid)) (fill none) (layer "Edge.Cuts"))
 (segment (start 142.1 103.1755) (end 141.825 103.4505) (width 0.25) (layer "F.Cu") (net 1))
 (segment (start 141.825 103.4505) (end 141.825 106.425) (width 0.25) (layer "F.Cu") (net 1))
 (segment (start 162.625 99.575) (end 163.625 98.575) (width 0.25) (layer "F.Cu") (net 1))
 (segment (start 125.4975 88.9) (end 132.08 88.9) (width 0.25) (layer "F.Cu") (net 1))
 (segment (start 150.9 106.425) (end 157.75 99.575) (width 0.25) (layer "F.Cu") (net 1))
 (segment (start 150.9 104) (end 151 103.9) (width 0.25) (layer "F.Cu") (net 1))
 (segment (start 124.46 89.9375) (end 106.8225 72.3) (width 0.25) (layer "F.Cu") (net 1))
 (segment (start 124.46 89.9375) (end 125.4975 88.9) (width 0.25) (layer "F.Cu") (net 1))
 (segment (start 128.75 94.2275) (end 124.46 89.9375) (width 0.25) (layer "F.Cu") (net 1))
 (segment (start 106.8225 72.3) (end 93.2 72.3) (width 0.25) (layer "F.Cu") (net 1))
 (segment (start 157.75 99.575) (end 162.625 99.575) (width 0.25) (layer "F.Cu") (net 1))
 (segment (start 128.75 106.425) (end 129.75 107.425) (width 0.25) (layer "F.Cu") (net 1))
 (segment (start 128.75 106.425) (end 128.75 94.2275) (width 0.25) (layer "F.Cu") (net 1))
 (segment (start 129.75 107.425) (end 140.825 107.425) (width 0.25) (layer "F.Cu") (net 1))
 (segment (start 140.825 107.425) (end 141.825 106.425) (width 0.25) (layer "F.Cu") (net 1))
 (segment (start 150.9 106.425) (end 150.9 104) (width 0.25) (layer "F.Cu") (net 1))
 (via (at 151 103.9) (size 0.8) (drill 0.4) (layers "F.Cu" "B.Cu") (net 1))
 (via (at 142.1 103.1755) (size 0.8) (drill 0.4) (layers "F.Cu" "B.Cu") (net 1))
 (segment (start 142.1005 103.175) (end 142.1 103.1755) (width 0.25) (layer "B.Cu") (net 1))
 (segment (start 150.275 103.175) (end 142.1005 103.175) (width 0.25) (layer "B.Cu") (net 1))
 (segment (start 151 103.9) (end 150.275 103.175) (width 0.25) (layer "B.Cu") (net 1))
 (segment (start 134.12 95.22) (end 134.1 95.2) (width 0.25) (layer "F.Cu") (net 4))
 (segment (start 156.9 106.425) (end 156.9 104.8) (width 0.25) (layer "F.Cu") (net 4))
 (segment (start 124.46 87.8625) (end 124.7375 87.8625) (width 0.25) (layer "F.Cu") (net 4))
 (segment (start 138.75 103.75) (end 138.7 103.7) (width 0.25) (layer "F.Cu") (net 4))
 (segment (start 134.12 96.52) (end 134.12 95.22) (width 0.25) (layer "F.Cu") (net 4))
 (segment (start 126.36 86.36) (end 126.3 86.3) (width 0.25) (layer "F.Cu") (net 4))
 (segment (start 124.7375 87.8625) (end 126.3 86.3) (width 0.25) (layer "F.Cu") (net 4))
 (segment (start 147.825 106.425) (end 147.825 104.075) (width 0.25) (layer "F.Cu") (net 4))
 (segment (start 147.825 104.075) (end 148 103.9) (width 0.25) (layer "F.Cu") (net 4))
 (segment (start 146.3 72.5) (end 146.3 74.1) (width 0.25) (layer "F.Cu") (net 4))
 (segment (start 128.5025 86.36) (end 126.36 86.36) (width 0.25) (layer "F.Cu") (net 4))
 (segment (start 138.75 106.425) (end 138.75 103.75) (width 0.25) (layer "F.Cu") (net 4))
 (segment (start 146.3 74.1) (end 146 74.4) (width 0.25) (layer "F.Cu") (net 4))
 (segment (start 132.08 89.85) (end 129.65 89.85) (width 0.25) (layer "F.Cu") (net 4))
 (segment (start 129.65 89.85) (end 129.6 89.8) (width 0.25) (layer "F.Cu") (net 4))
 (via (at 156.9 104.8) (size 0.8) (drill 0.4) (layers "F.Cu" "B.Cu") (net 4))
 (via (at 138.7 103.7) (size 0.8) (drill 0.4) (layers "F.Cu" "B.Cu") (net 4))
 (via (at 134.1 95.2) (size 0.8) (drill 0.4) (layers "F.Cu" "B.Cu") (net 4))
 (via (at 148 103.9) (size 0.8) (drill 0.4) (layers "F.Cu" "B.Cu") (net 4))
 (via (at 146 74.4) (size 0.8) (drill 0.4) (layers "F.Cu" "B.Cu") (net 4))
 (via (at 126.3 86.3) (size 0.8) (drill 0.4) (layers "F.Cu" "B.Cu") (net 4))
 (via (at 129.6 89.8) (size 0.8) (drill 0.4) (layers "F.Cu" "B.Cu") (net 4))
 (segment (start 130.6 89.8) (end 129.6 89.8) (width 0.25) (layer "B.Cu") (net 4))
 (segment (start 126.3 86.3) (end 117.325 77.325) (width 0.25) (layer "B.Cu") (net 4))
 (segment (start 148 103.9) (end 138.9 103.9) (width 0.25) (layer "B.Cu") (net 4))
 (segment (start 134.1 95.2) (end 134.1 94.3) (width 0.25) (layer "B.Cu") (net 4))
 (segment (start 148 103.9) (end 148.9 104.8) (width 0.25) (layer "B.Cu") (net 4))
 (segment (start 115.325 72.275) (end 95.225 72.275) (width 0.25) (layer "B.Cu") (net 4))
 (segment (start 134.1 95.2) (end 134.1 99.1) (width 0.25) (layer "B.Cu") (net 4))
 (segment (start 95.225 72.275) (end 93.2 74.3) (width 0.25) (layer "B.Cu") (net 4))
 (segment (start 159.4 104.8) (end 163.625 100.575) (width 0.25) (layer "B.Cu") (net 4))
 (segment (start 138.9 103.9) (end 138.7 103.7) (width 0.25) (layer "B.Cu") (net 4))
 (segment (start 134.1 99.1) (end 138.7 103.7) (width 0.25) (layer "B.Cu") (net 4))
 (segment (start 129.6 89.8) (end 126.3 86.5) (width 0.25) (layer "B.Cu") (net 4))
 (segment (start 115.325 72.275) (end 117.325 72.275) (width 0.25) (layer "B.Cu") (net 4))
 (segment (start 148.9 104.8) (end 156.9 104.8) (width 0.25) (layer "B.Cu") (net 4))
 (segment (start 134.1 94.3) (end 129.6 89.8) (width 0.25) (layer "B.Cu") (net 4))
 (segment (start 156.9 104.8) (end 159.4 104.8) (width 0.25) (layer "B.Cu") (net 4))
 (segment (start 126.3 86.5) (end 126.3 86.3) (width 0.25) (layer "B.Cu") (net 4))
 (segment (start 146 74.4) (end 130.6 89.8) (width 0.25) (layer "B.Cu") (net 4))
 (segment (start 117.325 77.325) (end 117.325 72.275) (width 0.25) (layer "B.Cu") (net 4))
 (segment (start 134.355 88.9) (end 131.815 86.36) (width 0.25) (layer "F.Cu") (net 7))
 (segment (start 130.5775 81.5275) (end 121.325 72.275) (width 0.25) (layer "F.Cu") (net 7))
 (segment (start 133.62 96.52) (end 133.62 95.745305) (width 0.25) (layer "F.Cu") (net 7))
 (segment (start 134.355 88.9) (end 139.9 88.9) (width 0.25) (layer "F.Cu") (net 7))
 (segment (start 139.9 88.9) (end 156.3 72.5) (width 0.25) (layer "F.Cu") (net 7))
 (segment (start 131.815 86.36) (end 130.5775 86.36) (width 0.25) (layer "F.Cu") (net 7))
 (segment (start 133.62 95.745305) (end 133.3675 95.492805) (width 0.25) (layer "F.Cu") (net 7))
 (segment (start 133.3675 95.492805) (end 133.3675 89.8875) (width 0.25) (layer "F.Cu") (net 7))
 (segment (start 133.3675 89.8875) (end 134.355 88.9) (width 0.25) (layer "F.Cu") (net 7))
 (segment (start 119.325 72.275) (end 121.325 72.275) (width 0.25) (layer "F.Cu") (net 7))
 (segment (start 130.5775 86.36) (end 130.5775 81.5275) (width 0.25) (layer "F.Cu") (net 7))
 (segment (start 152.9 106.425) (end 151.9 107.425) (width 0.25) (layer "F.Cu") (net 2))
 (segment (start 149.9 102.85) (end 160.175 92.575) (width 0.25) (layer "F.Cu") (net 2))
 (segment (start 151.9 107.425) (end 149.9 107.425) (width 0.25) (layer "F.Cu") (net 2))
 (segment (start 149.9 107.425) (end 149.9 102.85) (width 0.25) (layer "F.Cu") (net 2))
 (segment (start 149.45 101.3) (end 160.175 90.575) (width 0.25) (layer "F.Cu") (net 3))
 (segment (start 149.713604 107.875) (end 149.45 107.611396) (width 0.25) (layer "F.Cu") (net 3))
 (segment (start 154.9 106.425) (end 153.45 107.875) (width 0.25) (layer "F.Cu") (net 3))
 (segment (start 153.45 107.875) (end 149.713604 107.875) (width 0.25) (layer "F.Cu") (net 3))
 (segment (start 149.45 107.611396) (end 149.45 101.3) (width 0.25) (layer "F.Cu") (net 3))
 (segment (start 160.15 106.425) (end 160.15 100.6) (width 0.25) (layer "F.Cu") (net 23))
 (segment (start 160.15 100.6) (end 160.175 100.575) (width 0.25) (layer "F.Cu") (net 23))
 (segment (start 123.325 72.275) (end 125.325 72.275) (width 0.25) (layer "F.Cu") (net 12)))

